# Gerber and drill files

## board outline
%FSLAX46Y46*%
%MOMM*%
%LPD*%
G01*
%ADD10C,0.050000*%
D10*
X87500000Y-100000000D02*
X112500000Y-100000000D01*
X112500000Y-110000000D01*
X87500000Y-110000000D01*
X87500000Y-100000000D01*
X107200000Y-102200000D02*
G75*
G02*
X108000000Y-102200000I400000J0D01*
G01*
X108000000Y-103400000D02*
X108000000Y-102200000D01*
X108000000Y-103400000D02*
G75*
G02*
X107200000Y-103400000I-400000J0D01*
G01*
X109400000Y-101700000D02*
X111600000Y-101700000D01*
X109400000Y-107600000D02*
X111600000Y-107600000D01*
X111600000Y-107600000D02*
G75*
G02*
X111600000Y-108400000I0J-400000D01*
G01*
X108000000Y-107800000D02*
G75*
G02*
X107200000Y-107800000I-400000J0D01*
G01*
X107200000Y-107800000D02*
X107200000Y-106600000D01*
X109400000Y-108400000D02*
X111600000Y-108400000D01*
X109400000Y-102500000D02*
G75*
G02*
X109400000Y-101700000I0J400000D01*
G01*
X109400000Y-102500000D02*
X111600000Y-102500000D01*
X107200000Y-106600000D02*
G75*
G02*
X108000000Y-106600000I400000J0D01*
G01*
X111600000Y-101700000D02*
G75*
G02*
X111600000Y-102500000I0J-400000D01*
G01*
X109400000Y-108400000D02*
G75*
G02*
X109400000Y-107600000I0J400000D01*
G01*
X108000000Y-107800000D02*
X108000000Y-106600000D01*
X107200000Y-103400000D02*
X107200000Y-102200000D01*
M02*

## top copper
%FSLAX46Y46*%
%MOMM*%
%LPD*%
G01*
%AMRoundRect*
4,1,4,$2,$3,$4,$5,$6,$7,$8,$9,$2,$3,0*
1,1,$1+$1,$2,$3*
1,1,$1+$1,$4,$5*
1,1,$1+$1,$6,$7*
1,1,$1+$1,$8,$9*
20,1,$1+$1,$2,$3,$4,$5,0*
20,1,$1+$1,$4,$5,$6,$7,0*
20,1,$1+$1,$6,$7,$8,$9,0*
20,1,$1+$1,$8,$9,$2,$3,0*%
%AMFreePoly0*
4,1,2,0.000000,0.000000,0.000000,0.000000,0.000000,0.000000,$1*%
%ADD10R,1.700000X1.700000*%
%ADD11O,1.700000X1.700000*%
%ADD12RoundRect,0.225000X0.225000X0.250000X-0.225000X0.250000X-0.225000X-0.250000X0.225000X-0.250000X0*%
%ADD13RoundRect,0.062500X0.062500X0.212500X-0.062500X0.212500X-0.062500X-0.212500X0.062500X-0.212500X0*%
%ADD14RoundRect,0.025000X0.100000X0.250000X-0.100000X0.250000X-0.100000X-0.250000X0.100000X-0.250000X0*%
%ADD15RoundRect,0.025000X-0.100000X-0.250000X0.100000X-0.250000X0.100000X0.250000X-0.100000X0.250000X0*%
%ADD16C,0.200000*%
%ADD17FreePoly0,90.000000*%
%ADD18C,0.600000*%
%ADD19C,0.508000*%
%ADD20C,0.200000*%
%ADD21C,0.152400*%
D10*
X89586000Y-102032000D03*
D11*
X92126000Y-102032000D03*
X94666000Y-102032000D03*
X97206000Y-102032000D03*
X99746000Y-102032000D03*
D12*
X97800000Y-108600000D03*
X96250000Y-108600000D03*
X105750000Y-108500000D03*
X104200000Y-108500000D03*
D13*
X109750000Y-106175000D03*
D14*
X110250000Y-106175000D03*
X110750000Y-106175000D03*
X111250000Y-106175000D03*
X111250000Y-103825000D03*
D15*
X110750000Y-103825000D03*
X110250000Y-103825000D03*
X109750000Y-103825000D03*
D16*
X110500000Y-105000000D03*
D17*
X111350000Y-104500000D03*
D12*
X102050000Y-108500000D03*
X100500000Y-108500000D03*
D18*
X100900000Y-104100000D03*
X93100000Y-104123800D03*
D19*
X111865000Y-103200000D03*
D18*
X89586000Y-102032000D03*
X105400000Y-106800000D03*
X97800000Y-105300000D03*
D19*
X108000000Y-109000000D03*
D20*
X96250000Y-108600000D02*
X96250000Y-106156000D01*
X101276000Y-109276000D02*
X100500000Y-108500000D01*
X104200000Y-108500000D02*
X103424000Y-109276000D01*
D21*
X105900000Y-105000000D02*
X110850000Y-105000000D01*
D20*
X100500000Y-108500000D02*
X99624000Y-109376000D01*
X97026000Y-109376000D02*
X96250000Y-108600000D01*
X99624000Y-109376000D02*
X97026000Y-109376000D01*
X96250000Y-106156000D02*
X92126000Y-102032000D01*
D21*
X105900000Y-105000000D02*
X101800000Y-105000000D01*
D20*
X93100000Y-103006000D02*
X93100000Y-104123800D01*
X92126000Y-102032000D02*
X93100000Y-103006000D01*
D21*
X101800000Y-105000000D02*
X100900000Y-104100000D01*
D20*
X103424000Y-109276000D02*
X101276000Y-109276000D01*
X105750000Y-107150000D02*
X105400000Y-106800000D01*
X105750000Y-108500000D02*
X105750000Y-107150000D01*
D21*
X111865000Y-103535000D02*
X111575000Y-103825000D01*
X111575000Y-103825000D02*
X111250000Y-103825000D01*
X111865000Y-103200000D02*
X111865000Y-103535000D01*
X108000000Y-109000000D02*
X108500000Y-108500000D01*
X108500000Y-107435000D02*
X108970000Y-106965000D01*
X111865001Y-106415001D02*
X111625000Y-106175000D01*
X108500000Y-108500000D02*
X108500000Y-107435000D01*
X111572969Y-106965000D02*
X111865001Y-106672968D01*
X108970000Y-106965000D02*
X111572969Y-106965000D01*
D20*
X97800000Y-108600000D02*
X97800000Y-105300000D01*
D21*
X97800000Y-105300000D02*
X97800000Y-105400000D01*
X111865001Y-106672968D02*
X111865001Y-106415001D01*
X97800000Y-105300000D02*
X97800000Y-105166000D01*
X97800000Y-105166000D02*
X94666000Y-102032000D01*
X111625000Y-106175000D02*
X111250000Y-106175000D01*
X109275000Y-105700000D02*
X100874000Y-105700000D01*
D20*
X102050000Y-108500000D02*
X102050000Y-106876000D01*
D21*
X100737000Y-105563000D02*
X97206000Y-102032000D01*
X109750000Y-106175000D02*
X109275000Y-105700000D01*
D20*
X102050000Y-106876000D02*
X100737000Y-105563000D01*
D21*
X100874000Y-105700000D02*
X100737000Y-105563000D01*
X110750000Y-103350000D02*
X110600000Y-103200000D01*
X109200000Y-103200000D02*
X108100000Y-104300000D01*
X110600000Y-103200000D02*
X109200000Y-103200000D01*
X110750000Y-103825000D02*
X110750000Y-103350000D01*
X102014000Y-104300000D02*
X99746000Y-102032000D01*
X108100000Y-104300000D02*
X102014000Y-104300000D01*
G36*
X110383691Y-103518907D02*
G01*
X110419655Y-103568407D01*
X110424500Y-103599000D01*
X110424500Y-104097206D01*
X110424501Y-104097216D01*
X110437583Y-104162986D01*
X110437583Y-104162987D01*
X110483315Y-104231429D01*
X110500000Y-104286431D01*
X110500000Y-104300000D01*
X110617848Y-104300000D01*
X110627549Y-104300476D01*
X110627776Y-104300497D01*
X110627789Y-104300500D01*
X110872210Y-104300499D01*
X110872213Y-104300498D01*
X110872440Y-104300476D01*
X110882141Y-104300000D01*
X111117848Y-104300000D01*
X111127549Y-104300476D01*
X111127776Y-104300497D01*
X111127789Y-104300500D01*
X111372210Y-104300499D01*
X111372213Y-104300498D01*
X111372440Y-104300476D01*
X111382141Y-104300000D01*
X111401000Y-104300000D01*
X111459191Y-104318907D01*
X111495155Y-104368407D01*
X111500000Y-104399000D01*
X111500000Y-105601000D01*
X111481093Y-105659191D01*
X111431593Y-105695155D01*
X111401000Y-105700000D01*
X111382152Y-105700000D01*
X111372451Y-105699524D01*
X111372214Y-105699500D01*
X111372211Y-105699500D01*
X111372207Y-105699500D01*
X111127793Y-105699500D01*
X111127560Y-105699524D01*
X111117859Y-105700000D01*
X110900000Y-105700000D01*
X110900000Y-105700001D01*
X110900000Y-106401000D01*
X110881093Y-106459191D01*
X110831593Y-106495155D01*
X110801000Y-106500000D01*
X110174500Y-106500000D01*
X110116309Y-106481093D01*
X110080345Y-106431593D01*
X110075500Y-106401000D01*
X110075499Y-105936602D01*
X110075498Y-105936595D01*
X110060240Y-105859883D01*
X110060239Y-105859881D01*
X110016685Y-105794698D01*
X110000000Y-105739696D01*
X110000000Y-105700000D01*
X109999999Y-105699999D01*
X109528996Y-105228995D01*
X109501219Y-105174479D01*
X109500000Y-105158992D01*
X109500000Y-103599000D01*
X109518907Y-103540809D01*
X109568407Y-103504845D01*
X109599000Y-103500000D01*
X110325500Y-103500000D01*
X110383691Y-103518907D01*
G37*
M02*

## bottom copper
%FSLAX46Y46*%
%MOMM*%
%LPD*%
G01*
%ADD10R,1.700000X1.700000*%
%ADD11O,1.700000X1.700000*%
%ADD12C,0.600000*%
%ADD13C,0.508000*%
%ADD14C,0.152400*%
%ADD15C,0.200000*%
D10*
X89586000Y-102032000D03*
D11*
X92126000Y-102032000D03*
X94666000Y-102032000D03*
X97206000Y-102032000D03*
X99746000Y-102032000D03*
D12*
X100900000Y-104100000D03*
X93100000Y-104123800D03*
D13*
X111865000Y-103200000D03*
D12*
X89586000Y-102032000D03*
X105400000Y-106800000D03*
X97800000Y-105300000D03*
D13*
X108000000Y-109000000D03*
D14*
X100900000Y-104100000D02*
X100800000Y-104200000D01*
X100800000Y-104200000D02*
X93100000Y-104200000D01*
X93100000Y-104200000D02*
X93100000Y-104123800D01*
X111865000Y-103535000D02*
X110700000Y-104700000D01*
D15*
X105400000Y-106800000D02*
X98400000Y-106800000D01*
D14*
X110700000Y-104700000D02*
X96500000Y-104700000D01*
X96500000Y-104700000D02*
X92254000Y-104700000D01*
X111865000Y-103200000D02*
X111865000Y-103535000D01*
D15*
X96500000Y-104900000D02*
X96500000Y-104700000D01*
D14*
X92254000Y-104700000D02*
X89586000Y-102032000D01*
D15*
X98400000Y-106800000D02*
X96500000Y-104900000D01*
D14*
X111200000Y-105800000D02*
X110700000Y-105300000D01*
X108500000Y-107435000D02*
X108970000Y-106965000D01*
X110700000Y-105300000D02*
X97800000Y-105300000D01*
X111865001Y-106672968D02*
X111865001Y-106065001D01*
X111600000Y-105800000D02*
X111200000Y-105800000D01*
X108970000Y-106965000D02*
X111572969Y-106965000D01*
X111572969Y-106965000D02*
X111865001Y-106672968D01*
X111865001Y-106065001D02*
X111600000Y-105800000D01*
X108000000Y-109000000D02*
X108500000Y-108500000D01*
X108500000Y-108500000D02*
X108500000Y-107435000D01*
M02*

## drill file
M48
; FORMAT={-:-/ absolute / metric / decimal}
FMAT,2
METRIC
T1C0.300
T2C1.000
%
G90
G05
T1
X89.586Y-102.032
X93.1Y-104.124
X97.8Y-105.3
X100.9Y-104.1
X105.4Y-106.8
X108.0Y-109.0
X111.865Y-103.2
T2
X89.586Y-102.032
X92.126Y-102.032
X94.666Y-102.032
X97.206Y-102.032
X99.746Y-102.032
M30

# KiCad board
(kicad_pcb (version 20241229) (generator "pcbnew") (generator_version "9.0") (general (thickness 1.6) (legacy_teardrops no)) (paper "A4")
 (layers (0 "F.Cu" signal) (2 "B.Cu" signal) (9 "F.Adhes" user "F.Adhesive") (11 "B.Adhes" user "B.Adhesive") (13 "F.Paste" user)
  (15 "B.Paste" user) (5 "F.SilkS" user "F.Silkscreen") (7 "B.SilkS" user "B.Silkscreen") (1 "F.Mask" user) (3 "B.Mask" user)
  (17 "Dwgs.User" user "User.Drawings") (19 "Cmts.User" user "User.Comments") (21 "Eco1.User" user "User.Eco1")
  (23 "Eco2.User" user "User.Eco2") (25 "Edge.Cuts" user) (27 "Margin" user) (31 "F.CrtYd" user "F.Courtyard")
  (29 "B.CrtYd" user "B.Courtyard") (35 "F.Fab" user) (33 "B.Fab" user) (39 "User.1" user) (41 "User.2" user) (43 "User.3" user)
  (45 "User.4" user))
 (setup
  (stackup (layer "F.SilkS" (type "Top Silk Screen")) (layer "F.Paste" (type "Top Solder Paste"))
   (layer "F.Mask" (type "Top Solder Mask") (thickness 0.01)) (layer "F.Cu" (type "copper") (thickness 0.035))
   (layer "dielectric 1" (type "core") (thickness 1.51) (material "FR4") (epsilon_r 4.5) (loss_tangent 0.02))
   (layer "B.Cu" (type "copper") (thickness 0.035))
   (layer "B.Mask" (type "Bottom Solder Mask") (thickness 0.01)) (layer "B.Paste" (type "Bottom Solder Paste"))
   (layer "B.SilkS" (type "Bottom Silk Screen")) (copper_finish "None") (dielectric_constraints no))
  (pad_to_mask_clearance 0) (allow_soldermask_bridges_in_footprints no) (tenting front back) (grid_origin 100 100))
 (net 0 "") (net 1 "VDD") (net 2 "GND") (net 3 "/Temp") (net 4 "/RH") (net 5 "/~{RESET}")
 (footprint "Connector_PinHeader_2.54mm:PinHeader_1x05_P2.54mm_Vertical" (layer "F.Cu") (at 89.586 102.032 90)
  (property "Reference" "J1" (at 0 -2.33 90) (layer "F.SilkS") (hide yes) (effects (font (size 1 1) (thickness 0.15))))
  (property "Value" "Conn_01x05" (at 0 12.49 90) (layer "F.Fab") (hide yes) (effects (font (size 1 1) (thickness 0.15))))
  (pad "1" thru_hole rect (at 0 0 90) (size 1.7 1.7) (drill 1) (layers "*.Cu" "*.Mask") (remove_unused_layers no) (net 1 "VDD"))
  (pad "2" thru_hole oval (at 0 2.54 90) (size 1.7 1.7) (drill 1) (layers "*.Cu" "*.Mask") (remove_unused_layers no) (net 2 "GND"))
  (pad "3" thru_hole oval (at 0 5.08 90) (size 1.7 1.7) (drill 1) (layers "*.Cu" "*.Mask") (remove_unused_layers no) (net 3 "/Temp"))
  (pad "4" thru_hole oval (at 0 7.62 90) (size 1.7 1.7) (drill 1) (layers "*.Cu" "*.Mask") (remove_unused_layers no) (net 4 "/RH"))
  (pad "5" thru_hole oval (at 0 10.16 90) (size 1.7 1.7) (drill 1) (layers "*.Cu" "*.Mask") (remove_unused_layers no) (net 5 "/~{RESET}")))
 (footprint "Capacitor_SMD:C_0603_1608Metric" (layer "F.Cu") (at 97.025 108.6 180)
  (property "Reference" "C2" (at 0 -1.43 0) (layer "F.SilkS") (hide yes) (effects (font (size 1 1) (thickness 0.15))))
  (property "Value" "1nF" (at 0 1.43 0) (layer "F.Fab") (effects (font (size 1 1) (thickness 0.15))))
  (pad "1" smd roundrect (at -0.775 0 180) (size 0.9 0.95) (layers "F.Cu" "F.Mask" "F.Paste") (roundrect_rratio 0.25) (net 3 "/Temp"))
  (pad "2" smd roundrect (at 0.775 0 180) (size 0.9 0.95) (layers "F.Cu" "F.Mask" "F.Paste") (roundrect_rratio 0.25) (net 2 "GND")))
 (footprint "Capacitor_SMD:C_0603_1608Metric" (layer "F.Cu") (at 104.975 108.5 180)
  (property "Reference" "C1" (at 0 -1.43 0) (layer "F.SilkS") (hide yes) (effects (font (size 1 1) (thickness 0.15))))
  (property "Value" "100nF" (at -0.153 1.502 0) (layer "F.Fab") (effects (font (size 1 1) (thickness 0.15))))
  (pad "1" smd roundrect (at -0.775 0 180) (size 0.9 0.95) (layers "F.Cu" "F.Mask" "F.Paste") (roundrect_rratio 0.25) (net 1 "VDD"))
  (pad "2" smd roundrect (at 0.775 0 180) (size 0.9 0.95) (layers "F.Cu" "F.Mask" "F.Paste") (roundrect_rratio 0.25) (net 2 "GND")))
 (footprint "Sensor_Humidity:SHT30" (layer "F.Cu") (at 110.5 105 90)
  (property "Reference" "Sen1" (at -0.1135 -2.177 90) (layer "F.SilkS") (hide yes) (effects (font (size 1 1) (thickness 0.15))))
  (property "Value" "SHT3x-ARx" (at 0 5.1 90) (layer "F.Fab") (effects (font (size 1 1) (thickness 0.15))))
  (pad "1" smd roundrect (at -1.175 -0.75 180) (size 0.25 0.55) (layers "F.Cu" "F.Mask" "F.Paste") (roundrect_rratio 0.25) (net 4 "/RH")
   (solder_mask_margin 0.05) (solder_paste_margin 0))
  (pad "2" smd roundrect (at -1.175 -0.25 180) (size 0.25 0.55) (layers "F.Cu" "F.Mask" "F.Paste") (roundrect_rratio 0.1) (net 2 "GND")
   (solder_mask_margin 0.05) (solder_paste_margin 0))
  (pad "3" smd roundrect (at -1.175 0.25 180) (size 0.25 0.55) (layers "F.Cu" "F.Mask" "F.Paste") (roundrect_rratio 0.1) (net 2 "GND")
   (solder_mask_margin 0.05) (solder_paste_margin 0))
  (pad "4" smd roundrect (at -1.175 0.75 180) (size 0.25 0.55) (layers "F.Cu" "F.Mask" "F.Paste") (roundrect_rratio 0.1) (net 3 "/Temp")
   (solder_mask_margin 0.05) (solder_paste_margin 0))
  (pad "5" smd roundrect (at 1.175 0.75 180) (size 0.25 0.55) (layers "F.Cu" "F.Mask" "F.Paste") (roundrect_rratio 0.1) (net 1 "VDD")
   (solder_mask_margin 0.05) (solder_paste_margin 0))
  (pad "6" smd roundrect (at 1.175 0.25) (size 0.25 0.55) (layers "F.Cu" "F.Mask" "F.Paste") (roundrect_rratio 0.1) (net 5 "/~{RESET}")
   (solder_mask_margin 0.05) (solder_paste_margin 0))
  (pad "7" smd roundrect (at 1.175 -0.25) (size 0.25 0.55) (layers "F.Cu" "F.Mask" "F.Paste") (roundrect_rratio 0.1) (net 2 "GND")
   (solder_mask_margin 0.05) (solder_paste_margin 0))
  (pad "8" smd roundrect (at 1.175 -0.75) (size 0.25 0.55) (layers "F.Cu" "F.Mask" "F.Paste") (roundrect_rratio 0.1) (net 2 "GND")
   (solder_mask_margin 0.05) (solder_paste_margin 0))
  (pad "9" smd circle (at 0 0 270) (size 0.2 0.2) (layers "F.Cu" "F.Mask" "F.Paste") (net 2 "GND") (solder_mask_margin 0.05)
   (thermal_bridge_angle 90))
  (pad "9" smd custom (at 0.5 0.85 90) (size 0.000001 0.000001) (layers "F.Cu" "F.Mask" "F.Paste") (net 2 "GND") (solder_mask_margin 0.05)
   (solder_paste_margin -0.1) (thermal_bridge_angle 90) (options (clearance outline) (anchor circle)) (primitives)))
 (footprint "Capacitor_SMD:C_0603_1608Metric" (layer "F.Cu") (at 101.275 108.5 180)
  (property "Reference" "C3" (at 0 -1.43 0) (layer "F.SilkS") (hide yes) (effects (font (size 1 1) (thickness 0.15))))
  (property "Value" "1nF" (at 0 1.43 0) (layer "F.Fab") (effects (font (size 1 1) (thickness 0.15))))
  (pad "1" smd roundrect (at -0.775 0 180) (size 0.9 0.95) (layers "F.Cu" "F.Mask" "F.Paste") (roundrect_rratio 0.25) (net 4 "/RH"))
  (pad "2" smd roundrect (at 0.775 0 180) (size 0.9 0.95) (layers "F.Cu" "F.Mask" "F.Paste") (roundrect_rratio 0.25) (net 2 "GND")))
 (gr_rect (start 87.5 100) (end 112.5 110) (stroke (width 0.05) (type default)) (fill no) (layer "Edge.Cuts"))
 (gr_arc (start 107.2 102.2) (mid 107.6 101.8) (end 108 102.2) (stroke (width 0.05) (type default)) (layer "Edge.Cuts"))
 (gr_line (start 108 103.4) (end 108 102.2) (stroke (width 0.05) (type default)) (layer "Edge.Cuts"))
 (gr_arc (start 108 103.4) (mid 107.6 103.8) (end 107.2 103.4) (stroke (width 0.05) (type default)) (layer "Edge.Cuts"))
 (gr_line (start 109.4 101.7) (end 111.6 101.7) (stroke (width 0.05) (type default)) (layer "Edge.Cuts"))
 (gr_line (start 109.4 107.6) (end 111.6 107.6) (stroke (width 0.05) (type default)) (layer "Edge.Cuts"))
 (gr_arc (start 111.6 107.6) (mid 112 108) (end 111.6 108.4) (stroke (width 0.05) (type default)) (layer "Edge.Cuts"))
 (gr_arc (start 108 107.8) (mid 107.6 108.2) (end 107.2 107.8) (stroke (width 0.05) (type default)) (layer "Edge.Cuts"))
 (gr_line (start 107.2 107.8) (end 107.2 106.6) (stroke (width 0.05) (type default)) (layer "Edge.Cuts"))
 (gr_line (start 109.4 108.4) (end 111.6 108.4) (stroke (width 0.05) (type default)) (layer "Edge.Cuts"))
 (gr_arc (start 109.4 102.5) (mid 109 102.1) (end 109.4 101.7) (stroke (width 0.05) (type default)) (layer "Edge.Cuts"))
 (gr_line (start 109.4 102.5) (end 111.6 102.5) (stroke (width 0.05) (type default)) (layer "Edge.Cuts"))
 (gr_arc (start 107.2 106.6) (mid 107.6 106.2) (end 108 106.6) (stroke (width 0.05) (type default)) (layer "Edge.Cuts"))
 (gr_arc (start 111.6 101.7) (mid 112 102.1) (end 111.6 102.5) (stroke (width 0.05) (type default)) (layer "Edge.Cuts"))
 (gr_arc (start 109.4 108.4) (mid 109 108) (end 109.4 107.6) (stroke (width 0.05) (type default)) (layer "Edge.Cuts"))
 (gr_line (start 108 107.8) (end 108 106.6) (stroke (width 0.05) (type default)) (layer "Edge.Cuts"))
 (gr_line (start 107.2 103.4) (end 107.2 102.2) (stroke (width 0.05) (type default)) (layer "Edge.Cuts"))
 (segment (start 96.25 108.6) (end 96.25 106.156) (width 0.2) (layer "F.Cu") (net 2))
 (segment (start 101.276 109.276) (end 100.5 108.5) (width 0.2) (layer "F.Cu") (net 2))
 (segment (start 104.2 108.5) (end 103.424 109.276) (width 0.2) (layer "F.Cu") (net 2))
 (segment (start 105.9 105) (end 110.85 105) (width 0.1524) (layer "F.Cu") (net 2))
 (segment (start 100.5 108.5) (end 99.624 109.376) (width 0.2) (layer "F.Cu") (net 2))
 (segment (start 97.026 109.376) (end 96.25 108.6) (width 0.2) (layer "F.Cu") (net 2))
 (segment (start 99.624 109.376) (end 97.026 109.376) (width 0.2) (layer "F.Cu") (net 2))
 (segment (start 96.25 106.156) (end 92.126 102.032) (width 0.2) (layer "F.Cu") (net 2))
 (segment (start 105.9 105) (end 101.8 105) (width 0.1524) (layer "F.Cu") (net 2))
 (segment (start 93.1 103.006) (end 93.1 104.1238) (width 0.2) (layer "F.Cu") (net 2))
 (segment (start 92.126 102.032) (end 93.1 103.006) (width 0.2) (layer "F.Cu") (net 2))
 (segment (start 101.8 105) (end 100.9 104.1) (width 0.1524) (layer "F.Cu") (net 2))
 (segment (start 103.424 109.276) (end 101.276 109.276) (width 0.2) (layer "F.Cu") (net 2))
 (via (at 100.9 104.1) (size 0.6) (drill 0.3) (layers "F.Cu" "B.Cu") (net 2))
 (via (at 93.1 104.1238) (size 0.6) (drill 0.3) (layers "F.Cu" "B.Cu") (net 2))
 (segment (start 100.9 104.1) (end 100.8 104.2) (width 0.1524) (layer "B.Cu") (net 2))
 (segment (start 100.8 104.2) (end 93.1 104.2) (width 0.1524) (layer "B.Cu") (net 2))
 (segment (start 93.1 104.2) (end 93.1 104.1238) (width 0.1524) (layer "B.Cu") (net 2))
 (segment (start 105.75 107.15) (end 105.4 106.8) (width 0.2) (layer "F.Cu") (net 1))
 (segment (start 105.75 108.5) (end 105.75 107.15) (width 0.2) (layer "F.Cu") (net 1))
 (segment (start 111.865 103.535) (end 111.575 103.825) (width 0.1524) (layer "F.Cu") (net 1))
 (segment (start 111.575 103.825) (end 111.25 103.825) (width 0.1524) (layer "F.Cu") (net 1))
 (segment (start 111.865 103.2) (end 111.865 103.535) (width 0.1524) (layer "F.Cu") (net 1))
 (via (at 111.865 103.2) (size 0.508) (drill 0.3) (layers "F.Cu" "B.Cu")
  (teardrops (best_length_ratio 0.5) (max_length 1) (best_width_ratio 1) (max_width 0.127) (curved_edges no) (filter_ratio 0.9) (enabled no)
   (allow_two_segments yes) (prefer_zone_connections yes))
  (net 1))
 (via (at 89.586 102.032) (size 0.6) (drill 0.3) (layers "F.Cu" "B.Cu") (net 1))
 (via (at 105.4 106.8) (size 0.6) (drill 0.3) (layers "F.Cu" "B.Cu") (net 1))
 (segment (start 111.865 103.535) (end 110.7 104.7) (width 0.1524) (layer "B.Cu") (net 1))
 (segment (start 105.4 106.8) (end 98.4 106.8) (width 0.2) (layer "B.Cu") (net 1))
 (segment (start 110.7 104.7) (end 96.5 104.7) (width 0.1524) (layer "B.Cu") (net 1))
 (segment (start 96.5 104.7) (end 92.254 104.7) (width 0.1524) (layer "B.Cu") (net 1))
 (segment (start 111.865 103.2) (end 111.865 103.535) (width 0.1524) (layer "B.Cu") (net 1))
 (segment (start 96.5 104.9) (end 96.5 104.7) (width 0.2) (layer "B.Cu") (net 1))
 (segment (start 92.254 104.7) (end 89.586 102.032) (width 0.1524) (layer "B.Cu") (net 1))
 (segment (start 98.4 106.8) (end 96.5 104.9) (width 0.2) (layer "B.Cu") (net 1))
 (segment (start 108 109) (end 108.5 108.5) (width 0.1524) (layer "F.Cu") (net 3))
 (segment (start 108.5 107.435) (end 108.97 106.965) (width 0.1524) (layer "F.Cu") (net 3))
 (segment (start 111.865001 106.415001) (end 111.625 106.175) (width 0.1524) (layer "F.Cu") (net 3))
 (segment (start 108.5 108.5) (end 108.5 107.435) (width 0.1524) (layer "F.Cu") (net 3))
 (segment (start 111.572969 106.965) (end 111.865001 106.672968) (width 0.1524) (layer "F.Cu") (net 3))
 (segment (start 108.97 106.965) (end 111.572969 106.965) (width 0.1524) (layer "F.Cu") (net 3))
 (segment (start 97.8 108.6) (end 97.8 105.3) (width 0.2) (layer "F.Cu") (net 3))
 (segment (start 97.8 105.3) (end 97.8 105.4) (width 0.1524) (layer "F.Cu") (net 3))
 (segment (start 111.865001 106.672968) (end 111.865001 106.415001) (width 0.1524) (layer "F.Cu") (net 3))
 (segment (start 97.8 105.3) (end 97.8 105.166) (width 0.1524) (layer "F.Cu") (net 3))
 (segment (start 97.8 105.166) (end 94.666 102.032) (width 0.1524) (layer "F.Cu") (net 3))
 (segment (start 111.625 106.175) (end 111.25 106.175) (width 0.1524) (layer "F.Cu") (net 3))
 (via (at 97.8 105.3) (size 0.6) (drill 0.3) (layers "F.Cu" "B.Cu") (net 3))
 (via (at 108 109) (size 0.508) (drill 0.3) (layers "F.Cu" "B.Cu") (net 3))
 (segment (start 111.2 105.8) (end 110.7 105.3) (width 0.1524) (layer "B.Cu") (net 3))
 (segment (start 108.5 107.435) (end 108.97 106.965) (width 0.1524) (layer "B.Cu") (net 3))
 (segment (start 110.7 105.3) (end 97.8 105.3) (width 0.1524) (layer "B.Cu") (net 3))
 (segment (start 111.865001 106.672968) (end 111.865001 106.065001) (width 0.1524) (layer "B.Cu") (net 3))
 (segment (start 111.6 105.8) (end 111.2 105.8) (width 0.1524) (layer "B.Cu") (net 3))
 (segment (start 108.97 106.965) (end 111.572969 106.965) (width 0.1524) (layer "B.Cu") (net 3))
 (segment (start 111.572969 106.965) (end 111.865001 106.672968) (width 0.1524) (layer "B.Cu") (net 3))
 (segment (start 111.865001 106.065001) (end 111.6 105.8) (width 0.1524) (layer "B.Cu") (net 3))
 (segment (start 108 109) (end 108.5 108.5) (width 0.1524) (layer "B.Cu") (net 3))
 (segment (start 108.5 108.5) (end 108.5 107.435) (width 0.1524) (layer "B.Cu") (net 3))
 (segment (start 109.275 105.7) (end 100.874 105.7) (width 0.1524) (layer "F.Cu") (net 4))
 (segment (start 102.05 108.5) (end 102.05 106.876) (width 0.2) (layer "F.Cu") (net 4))
 (segment (start 100.737 105.563) (end 97.206 102.032) (width 0.1524) (layer "F.Cu") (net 4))
 (segment (start 109.75 106.175) (end 109.275 105.7) (width 0.1524) (layer "F.Cu") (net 4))
 (segment (start 102.05 106.876) (end 100.737 105.563) (width 0.2) (layer "F.Cu") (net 4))
 (segment (start 100.874 105.7) (end 100.737 105.563) (width 0.1524) (layer "F.Cu") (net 4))
 (segment (start 110.75 103.35) (end 110.6 103.2) (width 0.1524) (layer "F.Cu") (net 5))
 (segment (start 109.2 103.2) (end 108.1 104.3) (width 0.1524) (layer "F.Cu") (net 5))
 (segment (start 110.6 103.2) (end 109.2 103.2) (width 0.1524) (layer "F.Cu") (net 5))
 (segment (start 110.75 103.825) (end 110.75 103.35) (width 0.1524) (layer "F.Cu") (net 5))
 (segment (start 102.014 104.3) (end 99.746 102.032) (width 0.1524) (layer "F.Cu") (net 5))
 (segment (start 108.1 104.3) (end 102.014 104.3) (width 0.1524) (layer "F.Cu") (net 5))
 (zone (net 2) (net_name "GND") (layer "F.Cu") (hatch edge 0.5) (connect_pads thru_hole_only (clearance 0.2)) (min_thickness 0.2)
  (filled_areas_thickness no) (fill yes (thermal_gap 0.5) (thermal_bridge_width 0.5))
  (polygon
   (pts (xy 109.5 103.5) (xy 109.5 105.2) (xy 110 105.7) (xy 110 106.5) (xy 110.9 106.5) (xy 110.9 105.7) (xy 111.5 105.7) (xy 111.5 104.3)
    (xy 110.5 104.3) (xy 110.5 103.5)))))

